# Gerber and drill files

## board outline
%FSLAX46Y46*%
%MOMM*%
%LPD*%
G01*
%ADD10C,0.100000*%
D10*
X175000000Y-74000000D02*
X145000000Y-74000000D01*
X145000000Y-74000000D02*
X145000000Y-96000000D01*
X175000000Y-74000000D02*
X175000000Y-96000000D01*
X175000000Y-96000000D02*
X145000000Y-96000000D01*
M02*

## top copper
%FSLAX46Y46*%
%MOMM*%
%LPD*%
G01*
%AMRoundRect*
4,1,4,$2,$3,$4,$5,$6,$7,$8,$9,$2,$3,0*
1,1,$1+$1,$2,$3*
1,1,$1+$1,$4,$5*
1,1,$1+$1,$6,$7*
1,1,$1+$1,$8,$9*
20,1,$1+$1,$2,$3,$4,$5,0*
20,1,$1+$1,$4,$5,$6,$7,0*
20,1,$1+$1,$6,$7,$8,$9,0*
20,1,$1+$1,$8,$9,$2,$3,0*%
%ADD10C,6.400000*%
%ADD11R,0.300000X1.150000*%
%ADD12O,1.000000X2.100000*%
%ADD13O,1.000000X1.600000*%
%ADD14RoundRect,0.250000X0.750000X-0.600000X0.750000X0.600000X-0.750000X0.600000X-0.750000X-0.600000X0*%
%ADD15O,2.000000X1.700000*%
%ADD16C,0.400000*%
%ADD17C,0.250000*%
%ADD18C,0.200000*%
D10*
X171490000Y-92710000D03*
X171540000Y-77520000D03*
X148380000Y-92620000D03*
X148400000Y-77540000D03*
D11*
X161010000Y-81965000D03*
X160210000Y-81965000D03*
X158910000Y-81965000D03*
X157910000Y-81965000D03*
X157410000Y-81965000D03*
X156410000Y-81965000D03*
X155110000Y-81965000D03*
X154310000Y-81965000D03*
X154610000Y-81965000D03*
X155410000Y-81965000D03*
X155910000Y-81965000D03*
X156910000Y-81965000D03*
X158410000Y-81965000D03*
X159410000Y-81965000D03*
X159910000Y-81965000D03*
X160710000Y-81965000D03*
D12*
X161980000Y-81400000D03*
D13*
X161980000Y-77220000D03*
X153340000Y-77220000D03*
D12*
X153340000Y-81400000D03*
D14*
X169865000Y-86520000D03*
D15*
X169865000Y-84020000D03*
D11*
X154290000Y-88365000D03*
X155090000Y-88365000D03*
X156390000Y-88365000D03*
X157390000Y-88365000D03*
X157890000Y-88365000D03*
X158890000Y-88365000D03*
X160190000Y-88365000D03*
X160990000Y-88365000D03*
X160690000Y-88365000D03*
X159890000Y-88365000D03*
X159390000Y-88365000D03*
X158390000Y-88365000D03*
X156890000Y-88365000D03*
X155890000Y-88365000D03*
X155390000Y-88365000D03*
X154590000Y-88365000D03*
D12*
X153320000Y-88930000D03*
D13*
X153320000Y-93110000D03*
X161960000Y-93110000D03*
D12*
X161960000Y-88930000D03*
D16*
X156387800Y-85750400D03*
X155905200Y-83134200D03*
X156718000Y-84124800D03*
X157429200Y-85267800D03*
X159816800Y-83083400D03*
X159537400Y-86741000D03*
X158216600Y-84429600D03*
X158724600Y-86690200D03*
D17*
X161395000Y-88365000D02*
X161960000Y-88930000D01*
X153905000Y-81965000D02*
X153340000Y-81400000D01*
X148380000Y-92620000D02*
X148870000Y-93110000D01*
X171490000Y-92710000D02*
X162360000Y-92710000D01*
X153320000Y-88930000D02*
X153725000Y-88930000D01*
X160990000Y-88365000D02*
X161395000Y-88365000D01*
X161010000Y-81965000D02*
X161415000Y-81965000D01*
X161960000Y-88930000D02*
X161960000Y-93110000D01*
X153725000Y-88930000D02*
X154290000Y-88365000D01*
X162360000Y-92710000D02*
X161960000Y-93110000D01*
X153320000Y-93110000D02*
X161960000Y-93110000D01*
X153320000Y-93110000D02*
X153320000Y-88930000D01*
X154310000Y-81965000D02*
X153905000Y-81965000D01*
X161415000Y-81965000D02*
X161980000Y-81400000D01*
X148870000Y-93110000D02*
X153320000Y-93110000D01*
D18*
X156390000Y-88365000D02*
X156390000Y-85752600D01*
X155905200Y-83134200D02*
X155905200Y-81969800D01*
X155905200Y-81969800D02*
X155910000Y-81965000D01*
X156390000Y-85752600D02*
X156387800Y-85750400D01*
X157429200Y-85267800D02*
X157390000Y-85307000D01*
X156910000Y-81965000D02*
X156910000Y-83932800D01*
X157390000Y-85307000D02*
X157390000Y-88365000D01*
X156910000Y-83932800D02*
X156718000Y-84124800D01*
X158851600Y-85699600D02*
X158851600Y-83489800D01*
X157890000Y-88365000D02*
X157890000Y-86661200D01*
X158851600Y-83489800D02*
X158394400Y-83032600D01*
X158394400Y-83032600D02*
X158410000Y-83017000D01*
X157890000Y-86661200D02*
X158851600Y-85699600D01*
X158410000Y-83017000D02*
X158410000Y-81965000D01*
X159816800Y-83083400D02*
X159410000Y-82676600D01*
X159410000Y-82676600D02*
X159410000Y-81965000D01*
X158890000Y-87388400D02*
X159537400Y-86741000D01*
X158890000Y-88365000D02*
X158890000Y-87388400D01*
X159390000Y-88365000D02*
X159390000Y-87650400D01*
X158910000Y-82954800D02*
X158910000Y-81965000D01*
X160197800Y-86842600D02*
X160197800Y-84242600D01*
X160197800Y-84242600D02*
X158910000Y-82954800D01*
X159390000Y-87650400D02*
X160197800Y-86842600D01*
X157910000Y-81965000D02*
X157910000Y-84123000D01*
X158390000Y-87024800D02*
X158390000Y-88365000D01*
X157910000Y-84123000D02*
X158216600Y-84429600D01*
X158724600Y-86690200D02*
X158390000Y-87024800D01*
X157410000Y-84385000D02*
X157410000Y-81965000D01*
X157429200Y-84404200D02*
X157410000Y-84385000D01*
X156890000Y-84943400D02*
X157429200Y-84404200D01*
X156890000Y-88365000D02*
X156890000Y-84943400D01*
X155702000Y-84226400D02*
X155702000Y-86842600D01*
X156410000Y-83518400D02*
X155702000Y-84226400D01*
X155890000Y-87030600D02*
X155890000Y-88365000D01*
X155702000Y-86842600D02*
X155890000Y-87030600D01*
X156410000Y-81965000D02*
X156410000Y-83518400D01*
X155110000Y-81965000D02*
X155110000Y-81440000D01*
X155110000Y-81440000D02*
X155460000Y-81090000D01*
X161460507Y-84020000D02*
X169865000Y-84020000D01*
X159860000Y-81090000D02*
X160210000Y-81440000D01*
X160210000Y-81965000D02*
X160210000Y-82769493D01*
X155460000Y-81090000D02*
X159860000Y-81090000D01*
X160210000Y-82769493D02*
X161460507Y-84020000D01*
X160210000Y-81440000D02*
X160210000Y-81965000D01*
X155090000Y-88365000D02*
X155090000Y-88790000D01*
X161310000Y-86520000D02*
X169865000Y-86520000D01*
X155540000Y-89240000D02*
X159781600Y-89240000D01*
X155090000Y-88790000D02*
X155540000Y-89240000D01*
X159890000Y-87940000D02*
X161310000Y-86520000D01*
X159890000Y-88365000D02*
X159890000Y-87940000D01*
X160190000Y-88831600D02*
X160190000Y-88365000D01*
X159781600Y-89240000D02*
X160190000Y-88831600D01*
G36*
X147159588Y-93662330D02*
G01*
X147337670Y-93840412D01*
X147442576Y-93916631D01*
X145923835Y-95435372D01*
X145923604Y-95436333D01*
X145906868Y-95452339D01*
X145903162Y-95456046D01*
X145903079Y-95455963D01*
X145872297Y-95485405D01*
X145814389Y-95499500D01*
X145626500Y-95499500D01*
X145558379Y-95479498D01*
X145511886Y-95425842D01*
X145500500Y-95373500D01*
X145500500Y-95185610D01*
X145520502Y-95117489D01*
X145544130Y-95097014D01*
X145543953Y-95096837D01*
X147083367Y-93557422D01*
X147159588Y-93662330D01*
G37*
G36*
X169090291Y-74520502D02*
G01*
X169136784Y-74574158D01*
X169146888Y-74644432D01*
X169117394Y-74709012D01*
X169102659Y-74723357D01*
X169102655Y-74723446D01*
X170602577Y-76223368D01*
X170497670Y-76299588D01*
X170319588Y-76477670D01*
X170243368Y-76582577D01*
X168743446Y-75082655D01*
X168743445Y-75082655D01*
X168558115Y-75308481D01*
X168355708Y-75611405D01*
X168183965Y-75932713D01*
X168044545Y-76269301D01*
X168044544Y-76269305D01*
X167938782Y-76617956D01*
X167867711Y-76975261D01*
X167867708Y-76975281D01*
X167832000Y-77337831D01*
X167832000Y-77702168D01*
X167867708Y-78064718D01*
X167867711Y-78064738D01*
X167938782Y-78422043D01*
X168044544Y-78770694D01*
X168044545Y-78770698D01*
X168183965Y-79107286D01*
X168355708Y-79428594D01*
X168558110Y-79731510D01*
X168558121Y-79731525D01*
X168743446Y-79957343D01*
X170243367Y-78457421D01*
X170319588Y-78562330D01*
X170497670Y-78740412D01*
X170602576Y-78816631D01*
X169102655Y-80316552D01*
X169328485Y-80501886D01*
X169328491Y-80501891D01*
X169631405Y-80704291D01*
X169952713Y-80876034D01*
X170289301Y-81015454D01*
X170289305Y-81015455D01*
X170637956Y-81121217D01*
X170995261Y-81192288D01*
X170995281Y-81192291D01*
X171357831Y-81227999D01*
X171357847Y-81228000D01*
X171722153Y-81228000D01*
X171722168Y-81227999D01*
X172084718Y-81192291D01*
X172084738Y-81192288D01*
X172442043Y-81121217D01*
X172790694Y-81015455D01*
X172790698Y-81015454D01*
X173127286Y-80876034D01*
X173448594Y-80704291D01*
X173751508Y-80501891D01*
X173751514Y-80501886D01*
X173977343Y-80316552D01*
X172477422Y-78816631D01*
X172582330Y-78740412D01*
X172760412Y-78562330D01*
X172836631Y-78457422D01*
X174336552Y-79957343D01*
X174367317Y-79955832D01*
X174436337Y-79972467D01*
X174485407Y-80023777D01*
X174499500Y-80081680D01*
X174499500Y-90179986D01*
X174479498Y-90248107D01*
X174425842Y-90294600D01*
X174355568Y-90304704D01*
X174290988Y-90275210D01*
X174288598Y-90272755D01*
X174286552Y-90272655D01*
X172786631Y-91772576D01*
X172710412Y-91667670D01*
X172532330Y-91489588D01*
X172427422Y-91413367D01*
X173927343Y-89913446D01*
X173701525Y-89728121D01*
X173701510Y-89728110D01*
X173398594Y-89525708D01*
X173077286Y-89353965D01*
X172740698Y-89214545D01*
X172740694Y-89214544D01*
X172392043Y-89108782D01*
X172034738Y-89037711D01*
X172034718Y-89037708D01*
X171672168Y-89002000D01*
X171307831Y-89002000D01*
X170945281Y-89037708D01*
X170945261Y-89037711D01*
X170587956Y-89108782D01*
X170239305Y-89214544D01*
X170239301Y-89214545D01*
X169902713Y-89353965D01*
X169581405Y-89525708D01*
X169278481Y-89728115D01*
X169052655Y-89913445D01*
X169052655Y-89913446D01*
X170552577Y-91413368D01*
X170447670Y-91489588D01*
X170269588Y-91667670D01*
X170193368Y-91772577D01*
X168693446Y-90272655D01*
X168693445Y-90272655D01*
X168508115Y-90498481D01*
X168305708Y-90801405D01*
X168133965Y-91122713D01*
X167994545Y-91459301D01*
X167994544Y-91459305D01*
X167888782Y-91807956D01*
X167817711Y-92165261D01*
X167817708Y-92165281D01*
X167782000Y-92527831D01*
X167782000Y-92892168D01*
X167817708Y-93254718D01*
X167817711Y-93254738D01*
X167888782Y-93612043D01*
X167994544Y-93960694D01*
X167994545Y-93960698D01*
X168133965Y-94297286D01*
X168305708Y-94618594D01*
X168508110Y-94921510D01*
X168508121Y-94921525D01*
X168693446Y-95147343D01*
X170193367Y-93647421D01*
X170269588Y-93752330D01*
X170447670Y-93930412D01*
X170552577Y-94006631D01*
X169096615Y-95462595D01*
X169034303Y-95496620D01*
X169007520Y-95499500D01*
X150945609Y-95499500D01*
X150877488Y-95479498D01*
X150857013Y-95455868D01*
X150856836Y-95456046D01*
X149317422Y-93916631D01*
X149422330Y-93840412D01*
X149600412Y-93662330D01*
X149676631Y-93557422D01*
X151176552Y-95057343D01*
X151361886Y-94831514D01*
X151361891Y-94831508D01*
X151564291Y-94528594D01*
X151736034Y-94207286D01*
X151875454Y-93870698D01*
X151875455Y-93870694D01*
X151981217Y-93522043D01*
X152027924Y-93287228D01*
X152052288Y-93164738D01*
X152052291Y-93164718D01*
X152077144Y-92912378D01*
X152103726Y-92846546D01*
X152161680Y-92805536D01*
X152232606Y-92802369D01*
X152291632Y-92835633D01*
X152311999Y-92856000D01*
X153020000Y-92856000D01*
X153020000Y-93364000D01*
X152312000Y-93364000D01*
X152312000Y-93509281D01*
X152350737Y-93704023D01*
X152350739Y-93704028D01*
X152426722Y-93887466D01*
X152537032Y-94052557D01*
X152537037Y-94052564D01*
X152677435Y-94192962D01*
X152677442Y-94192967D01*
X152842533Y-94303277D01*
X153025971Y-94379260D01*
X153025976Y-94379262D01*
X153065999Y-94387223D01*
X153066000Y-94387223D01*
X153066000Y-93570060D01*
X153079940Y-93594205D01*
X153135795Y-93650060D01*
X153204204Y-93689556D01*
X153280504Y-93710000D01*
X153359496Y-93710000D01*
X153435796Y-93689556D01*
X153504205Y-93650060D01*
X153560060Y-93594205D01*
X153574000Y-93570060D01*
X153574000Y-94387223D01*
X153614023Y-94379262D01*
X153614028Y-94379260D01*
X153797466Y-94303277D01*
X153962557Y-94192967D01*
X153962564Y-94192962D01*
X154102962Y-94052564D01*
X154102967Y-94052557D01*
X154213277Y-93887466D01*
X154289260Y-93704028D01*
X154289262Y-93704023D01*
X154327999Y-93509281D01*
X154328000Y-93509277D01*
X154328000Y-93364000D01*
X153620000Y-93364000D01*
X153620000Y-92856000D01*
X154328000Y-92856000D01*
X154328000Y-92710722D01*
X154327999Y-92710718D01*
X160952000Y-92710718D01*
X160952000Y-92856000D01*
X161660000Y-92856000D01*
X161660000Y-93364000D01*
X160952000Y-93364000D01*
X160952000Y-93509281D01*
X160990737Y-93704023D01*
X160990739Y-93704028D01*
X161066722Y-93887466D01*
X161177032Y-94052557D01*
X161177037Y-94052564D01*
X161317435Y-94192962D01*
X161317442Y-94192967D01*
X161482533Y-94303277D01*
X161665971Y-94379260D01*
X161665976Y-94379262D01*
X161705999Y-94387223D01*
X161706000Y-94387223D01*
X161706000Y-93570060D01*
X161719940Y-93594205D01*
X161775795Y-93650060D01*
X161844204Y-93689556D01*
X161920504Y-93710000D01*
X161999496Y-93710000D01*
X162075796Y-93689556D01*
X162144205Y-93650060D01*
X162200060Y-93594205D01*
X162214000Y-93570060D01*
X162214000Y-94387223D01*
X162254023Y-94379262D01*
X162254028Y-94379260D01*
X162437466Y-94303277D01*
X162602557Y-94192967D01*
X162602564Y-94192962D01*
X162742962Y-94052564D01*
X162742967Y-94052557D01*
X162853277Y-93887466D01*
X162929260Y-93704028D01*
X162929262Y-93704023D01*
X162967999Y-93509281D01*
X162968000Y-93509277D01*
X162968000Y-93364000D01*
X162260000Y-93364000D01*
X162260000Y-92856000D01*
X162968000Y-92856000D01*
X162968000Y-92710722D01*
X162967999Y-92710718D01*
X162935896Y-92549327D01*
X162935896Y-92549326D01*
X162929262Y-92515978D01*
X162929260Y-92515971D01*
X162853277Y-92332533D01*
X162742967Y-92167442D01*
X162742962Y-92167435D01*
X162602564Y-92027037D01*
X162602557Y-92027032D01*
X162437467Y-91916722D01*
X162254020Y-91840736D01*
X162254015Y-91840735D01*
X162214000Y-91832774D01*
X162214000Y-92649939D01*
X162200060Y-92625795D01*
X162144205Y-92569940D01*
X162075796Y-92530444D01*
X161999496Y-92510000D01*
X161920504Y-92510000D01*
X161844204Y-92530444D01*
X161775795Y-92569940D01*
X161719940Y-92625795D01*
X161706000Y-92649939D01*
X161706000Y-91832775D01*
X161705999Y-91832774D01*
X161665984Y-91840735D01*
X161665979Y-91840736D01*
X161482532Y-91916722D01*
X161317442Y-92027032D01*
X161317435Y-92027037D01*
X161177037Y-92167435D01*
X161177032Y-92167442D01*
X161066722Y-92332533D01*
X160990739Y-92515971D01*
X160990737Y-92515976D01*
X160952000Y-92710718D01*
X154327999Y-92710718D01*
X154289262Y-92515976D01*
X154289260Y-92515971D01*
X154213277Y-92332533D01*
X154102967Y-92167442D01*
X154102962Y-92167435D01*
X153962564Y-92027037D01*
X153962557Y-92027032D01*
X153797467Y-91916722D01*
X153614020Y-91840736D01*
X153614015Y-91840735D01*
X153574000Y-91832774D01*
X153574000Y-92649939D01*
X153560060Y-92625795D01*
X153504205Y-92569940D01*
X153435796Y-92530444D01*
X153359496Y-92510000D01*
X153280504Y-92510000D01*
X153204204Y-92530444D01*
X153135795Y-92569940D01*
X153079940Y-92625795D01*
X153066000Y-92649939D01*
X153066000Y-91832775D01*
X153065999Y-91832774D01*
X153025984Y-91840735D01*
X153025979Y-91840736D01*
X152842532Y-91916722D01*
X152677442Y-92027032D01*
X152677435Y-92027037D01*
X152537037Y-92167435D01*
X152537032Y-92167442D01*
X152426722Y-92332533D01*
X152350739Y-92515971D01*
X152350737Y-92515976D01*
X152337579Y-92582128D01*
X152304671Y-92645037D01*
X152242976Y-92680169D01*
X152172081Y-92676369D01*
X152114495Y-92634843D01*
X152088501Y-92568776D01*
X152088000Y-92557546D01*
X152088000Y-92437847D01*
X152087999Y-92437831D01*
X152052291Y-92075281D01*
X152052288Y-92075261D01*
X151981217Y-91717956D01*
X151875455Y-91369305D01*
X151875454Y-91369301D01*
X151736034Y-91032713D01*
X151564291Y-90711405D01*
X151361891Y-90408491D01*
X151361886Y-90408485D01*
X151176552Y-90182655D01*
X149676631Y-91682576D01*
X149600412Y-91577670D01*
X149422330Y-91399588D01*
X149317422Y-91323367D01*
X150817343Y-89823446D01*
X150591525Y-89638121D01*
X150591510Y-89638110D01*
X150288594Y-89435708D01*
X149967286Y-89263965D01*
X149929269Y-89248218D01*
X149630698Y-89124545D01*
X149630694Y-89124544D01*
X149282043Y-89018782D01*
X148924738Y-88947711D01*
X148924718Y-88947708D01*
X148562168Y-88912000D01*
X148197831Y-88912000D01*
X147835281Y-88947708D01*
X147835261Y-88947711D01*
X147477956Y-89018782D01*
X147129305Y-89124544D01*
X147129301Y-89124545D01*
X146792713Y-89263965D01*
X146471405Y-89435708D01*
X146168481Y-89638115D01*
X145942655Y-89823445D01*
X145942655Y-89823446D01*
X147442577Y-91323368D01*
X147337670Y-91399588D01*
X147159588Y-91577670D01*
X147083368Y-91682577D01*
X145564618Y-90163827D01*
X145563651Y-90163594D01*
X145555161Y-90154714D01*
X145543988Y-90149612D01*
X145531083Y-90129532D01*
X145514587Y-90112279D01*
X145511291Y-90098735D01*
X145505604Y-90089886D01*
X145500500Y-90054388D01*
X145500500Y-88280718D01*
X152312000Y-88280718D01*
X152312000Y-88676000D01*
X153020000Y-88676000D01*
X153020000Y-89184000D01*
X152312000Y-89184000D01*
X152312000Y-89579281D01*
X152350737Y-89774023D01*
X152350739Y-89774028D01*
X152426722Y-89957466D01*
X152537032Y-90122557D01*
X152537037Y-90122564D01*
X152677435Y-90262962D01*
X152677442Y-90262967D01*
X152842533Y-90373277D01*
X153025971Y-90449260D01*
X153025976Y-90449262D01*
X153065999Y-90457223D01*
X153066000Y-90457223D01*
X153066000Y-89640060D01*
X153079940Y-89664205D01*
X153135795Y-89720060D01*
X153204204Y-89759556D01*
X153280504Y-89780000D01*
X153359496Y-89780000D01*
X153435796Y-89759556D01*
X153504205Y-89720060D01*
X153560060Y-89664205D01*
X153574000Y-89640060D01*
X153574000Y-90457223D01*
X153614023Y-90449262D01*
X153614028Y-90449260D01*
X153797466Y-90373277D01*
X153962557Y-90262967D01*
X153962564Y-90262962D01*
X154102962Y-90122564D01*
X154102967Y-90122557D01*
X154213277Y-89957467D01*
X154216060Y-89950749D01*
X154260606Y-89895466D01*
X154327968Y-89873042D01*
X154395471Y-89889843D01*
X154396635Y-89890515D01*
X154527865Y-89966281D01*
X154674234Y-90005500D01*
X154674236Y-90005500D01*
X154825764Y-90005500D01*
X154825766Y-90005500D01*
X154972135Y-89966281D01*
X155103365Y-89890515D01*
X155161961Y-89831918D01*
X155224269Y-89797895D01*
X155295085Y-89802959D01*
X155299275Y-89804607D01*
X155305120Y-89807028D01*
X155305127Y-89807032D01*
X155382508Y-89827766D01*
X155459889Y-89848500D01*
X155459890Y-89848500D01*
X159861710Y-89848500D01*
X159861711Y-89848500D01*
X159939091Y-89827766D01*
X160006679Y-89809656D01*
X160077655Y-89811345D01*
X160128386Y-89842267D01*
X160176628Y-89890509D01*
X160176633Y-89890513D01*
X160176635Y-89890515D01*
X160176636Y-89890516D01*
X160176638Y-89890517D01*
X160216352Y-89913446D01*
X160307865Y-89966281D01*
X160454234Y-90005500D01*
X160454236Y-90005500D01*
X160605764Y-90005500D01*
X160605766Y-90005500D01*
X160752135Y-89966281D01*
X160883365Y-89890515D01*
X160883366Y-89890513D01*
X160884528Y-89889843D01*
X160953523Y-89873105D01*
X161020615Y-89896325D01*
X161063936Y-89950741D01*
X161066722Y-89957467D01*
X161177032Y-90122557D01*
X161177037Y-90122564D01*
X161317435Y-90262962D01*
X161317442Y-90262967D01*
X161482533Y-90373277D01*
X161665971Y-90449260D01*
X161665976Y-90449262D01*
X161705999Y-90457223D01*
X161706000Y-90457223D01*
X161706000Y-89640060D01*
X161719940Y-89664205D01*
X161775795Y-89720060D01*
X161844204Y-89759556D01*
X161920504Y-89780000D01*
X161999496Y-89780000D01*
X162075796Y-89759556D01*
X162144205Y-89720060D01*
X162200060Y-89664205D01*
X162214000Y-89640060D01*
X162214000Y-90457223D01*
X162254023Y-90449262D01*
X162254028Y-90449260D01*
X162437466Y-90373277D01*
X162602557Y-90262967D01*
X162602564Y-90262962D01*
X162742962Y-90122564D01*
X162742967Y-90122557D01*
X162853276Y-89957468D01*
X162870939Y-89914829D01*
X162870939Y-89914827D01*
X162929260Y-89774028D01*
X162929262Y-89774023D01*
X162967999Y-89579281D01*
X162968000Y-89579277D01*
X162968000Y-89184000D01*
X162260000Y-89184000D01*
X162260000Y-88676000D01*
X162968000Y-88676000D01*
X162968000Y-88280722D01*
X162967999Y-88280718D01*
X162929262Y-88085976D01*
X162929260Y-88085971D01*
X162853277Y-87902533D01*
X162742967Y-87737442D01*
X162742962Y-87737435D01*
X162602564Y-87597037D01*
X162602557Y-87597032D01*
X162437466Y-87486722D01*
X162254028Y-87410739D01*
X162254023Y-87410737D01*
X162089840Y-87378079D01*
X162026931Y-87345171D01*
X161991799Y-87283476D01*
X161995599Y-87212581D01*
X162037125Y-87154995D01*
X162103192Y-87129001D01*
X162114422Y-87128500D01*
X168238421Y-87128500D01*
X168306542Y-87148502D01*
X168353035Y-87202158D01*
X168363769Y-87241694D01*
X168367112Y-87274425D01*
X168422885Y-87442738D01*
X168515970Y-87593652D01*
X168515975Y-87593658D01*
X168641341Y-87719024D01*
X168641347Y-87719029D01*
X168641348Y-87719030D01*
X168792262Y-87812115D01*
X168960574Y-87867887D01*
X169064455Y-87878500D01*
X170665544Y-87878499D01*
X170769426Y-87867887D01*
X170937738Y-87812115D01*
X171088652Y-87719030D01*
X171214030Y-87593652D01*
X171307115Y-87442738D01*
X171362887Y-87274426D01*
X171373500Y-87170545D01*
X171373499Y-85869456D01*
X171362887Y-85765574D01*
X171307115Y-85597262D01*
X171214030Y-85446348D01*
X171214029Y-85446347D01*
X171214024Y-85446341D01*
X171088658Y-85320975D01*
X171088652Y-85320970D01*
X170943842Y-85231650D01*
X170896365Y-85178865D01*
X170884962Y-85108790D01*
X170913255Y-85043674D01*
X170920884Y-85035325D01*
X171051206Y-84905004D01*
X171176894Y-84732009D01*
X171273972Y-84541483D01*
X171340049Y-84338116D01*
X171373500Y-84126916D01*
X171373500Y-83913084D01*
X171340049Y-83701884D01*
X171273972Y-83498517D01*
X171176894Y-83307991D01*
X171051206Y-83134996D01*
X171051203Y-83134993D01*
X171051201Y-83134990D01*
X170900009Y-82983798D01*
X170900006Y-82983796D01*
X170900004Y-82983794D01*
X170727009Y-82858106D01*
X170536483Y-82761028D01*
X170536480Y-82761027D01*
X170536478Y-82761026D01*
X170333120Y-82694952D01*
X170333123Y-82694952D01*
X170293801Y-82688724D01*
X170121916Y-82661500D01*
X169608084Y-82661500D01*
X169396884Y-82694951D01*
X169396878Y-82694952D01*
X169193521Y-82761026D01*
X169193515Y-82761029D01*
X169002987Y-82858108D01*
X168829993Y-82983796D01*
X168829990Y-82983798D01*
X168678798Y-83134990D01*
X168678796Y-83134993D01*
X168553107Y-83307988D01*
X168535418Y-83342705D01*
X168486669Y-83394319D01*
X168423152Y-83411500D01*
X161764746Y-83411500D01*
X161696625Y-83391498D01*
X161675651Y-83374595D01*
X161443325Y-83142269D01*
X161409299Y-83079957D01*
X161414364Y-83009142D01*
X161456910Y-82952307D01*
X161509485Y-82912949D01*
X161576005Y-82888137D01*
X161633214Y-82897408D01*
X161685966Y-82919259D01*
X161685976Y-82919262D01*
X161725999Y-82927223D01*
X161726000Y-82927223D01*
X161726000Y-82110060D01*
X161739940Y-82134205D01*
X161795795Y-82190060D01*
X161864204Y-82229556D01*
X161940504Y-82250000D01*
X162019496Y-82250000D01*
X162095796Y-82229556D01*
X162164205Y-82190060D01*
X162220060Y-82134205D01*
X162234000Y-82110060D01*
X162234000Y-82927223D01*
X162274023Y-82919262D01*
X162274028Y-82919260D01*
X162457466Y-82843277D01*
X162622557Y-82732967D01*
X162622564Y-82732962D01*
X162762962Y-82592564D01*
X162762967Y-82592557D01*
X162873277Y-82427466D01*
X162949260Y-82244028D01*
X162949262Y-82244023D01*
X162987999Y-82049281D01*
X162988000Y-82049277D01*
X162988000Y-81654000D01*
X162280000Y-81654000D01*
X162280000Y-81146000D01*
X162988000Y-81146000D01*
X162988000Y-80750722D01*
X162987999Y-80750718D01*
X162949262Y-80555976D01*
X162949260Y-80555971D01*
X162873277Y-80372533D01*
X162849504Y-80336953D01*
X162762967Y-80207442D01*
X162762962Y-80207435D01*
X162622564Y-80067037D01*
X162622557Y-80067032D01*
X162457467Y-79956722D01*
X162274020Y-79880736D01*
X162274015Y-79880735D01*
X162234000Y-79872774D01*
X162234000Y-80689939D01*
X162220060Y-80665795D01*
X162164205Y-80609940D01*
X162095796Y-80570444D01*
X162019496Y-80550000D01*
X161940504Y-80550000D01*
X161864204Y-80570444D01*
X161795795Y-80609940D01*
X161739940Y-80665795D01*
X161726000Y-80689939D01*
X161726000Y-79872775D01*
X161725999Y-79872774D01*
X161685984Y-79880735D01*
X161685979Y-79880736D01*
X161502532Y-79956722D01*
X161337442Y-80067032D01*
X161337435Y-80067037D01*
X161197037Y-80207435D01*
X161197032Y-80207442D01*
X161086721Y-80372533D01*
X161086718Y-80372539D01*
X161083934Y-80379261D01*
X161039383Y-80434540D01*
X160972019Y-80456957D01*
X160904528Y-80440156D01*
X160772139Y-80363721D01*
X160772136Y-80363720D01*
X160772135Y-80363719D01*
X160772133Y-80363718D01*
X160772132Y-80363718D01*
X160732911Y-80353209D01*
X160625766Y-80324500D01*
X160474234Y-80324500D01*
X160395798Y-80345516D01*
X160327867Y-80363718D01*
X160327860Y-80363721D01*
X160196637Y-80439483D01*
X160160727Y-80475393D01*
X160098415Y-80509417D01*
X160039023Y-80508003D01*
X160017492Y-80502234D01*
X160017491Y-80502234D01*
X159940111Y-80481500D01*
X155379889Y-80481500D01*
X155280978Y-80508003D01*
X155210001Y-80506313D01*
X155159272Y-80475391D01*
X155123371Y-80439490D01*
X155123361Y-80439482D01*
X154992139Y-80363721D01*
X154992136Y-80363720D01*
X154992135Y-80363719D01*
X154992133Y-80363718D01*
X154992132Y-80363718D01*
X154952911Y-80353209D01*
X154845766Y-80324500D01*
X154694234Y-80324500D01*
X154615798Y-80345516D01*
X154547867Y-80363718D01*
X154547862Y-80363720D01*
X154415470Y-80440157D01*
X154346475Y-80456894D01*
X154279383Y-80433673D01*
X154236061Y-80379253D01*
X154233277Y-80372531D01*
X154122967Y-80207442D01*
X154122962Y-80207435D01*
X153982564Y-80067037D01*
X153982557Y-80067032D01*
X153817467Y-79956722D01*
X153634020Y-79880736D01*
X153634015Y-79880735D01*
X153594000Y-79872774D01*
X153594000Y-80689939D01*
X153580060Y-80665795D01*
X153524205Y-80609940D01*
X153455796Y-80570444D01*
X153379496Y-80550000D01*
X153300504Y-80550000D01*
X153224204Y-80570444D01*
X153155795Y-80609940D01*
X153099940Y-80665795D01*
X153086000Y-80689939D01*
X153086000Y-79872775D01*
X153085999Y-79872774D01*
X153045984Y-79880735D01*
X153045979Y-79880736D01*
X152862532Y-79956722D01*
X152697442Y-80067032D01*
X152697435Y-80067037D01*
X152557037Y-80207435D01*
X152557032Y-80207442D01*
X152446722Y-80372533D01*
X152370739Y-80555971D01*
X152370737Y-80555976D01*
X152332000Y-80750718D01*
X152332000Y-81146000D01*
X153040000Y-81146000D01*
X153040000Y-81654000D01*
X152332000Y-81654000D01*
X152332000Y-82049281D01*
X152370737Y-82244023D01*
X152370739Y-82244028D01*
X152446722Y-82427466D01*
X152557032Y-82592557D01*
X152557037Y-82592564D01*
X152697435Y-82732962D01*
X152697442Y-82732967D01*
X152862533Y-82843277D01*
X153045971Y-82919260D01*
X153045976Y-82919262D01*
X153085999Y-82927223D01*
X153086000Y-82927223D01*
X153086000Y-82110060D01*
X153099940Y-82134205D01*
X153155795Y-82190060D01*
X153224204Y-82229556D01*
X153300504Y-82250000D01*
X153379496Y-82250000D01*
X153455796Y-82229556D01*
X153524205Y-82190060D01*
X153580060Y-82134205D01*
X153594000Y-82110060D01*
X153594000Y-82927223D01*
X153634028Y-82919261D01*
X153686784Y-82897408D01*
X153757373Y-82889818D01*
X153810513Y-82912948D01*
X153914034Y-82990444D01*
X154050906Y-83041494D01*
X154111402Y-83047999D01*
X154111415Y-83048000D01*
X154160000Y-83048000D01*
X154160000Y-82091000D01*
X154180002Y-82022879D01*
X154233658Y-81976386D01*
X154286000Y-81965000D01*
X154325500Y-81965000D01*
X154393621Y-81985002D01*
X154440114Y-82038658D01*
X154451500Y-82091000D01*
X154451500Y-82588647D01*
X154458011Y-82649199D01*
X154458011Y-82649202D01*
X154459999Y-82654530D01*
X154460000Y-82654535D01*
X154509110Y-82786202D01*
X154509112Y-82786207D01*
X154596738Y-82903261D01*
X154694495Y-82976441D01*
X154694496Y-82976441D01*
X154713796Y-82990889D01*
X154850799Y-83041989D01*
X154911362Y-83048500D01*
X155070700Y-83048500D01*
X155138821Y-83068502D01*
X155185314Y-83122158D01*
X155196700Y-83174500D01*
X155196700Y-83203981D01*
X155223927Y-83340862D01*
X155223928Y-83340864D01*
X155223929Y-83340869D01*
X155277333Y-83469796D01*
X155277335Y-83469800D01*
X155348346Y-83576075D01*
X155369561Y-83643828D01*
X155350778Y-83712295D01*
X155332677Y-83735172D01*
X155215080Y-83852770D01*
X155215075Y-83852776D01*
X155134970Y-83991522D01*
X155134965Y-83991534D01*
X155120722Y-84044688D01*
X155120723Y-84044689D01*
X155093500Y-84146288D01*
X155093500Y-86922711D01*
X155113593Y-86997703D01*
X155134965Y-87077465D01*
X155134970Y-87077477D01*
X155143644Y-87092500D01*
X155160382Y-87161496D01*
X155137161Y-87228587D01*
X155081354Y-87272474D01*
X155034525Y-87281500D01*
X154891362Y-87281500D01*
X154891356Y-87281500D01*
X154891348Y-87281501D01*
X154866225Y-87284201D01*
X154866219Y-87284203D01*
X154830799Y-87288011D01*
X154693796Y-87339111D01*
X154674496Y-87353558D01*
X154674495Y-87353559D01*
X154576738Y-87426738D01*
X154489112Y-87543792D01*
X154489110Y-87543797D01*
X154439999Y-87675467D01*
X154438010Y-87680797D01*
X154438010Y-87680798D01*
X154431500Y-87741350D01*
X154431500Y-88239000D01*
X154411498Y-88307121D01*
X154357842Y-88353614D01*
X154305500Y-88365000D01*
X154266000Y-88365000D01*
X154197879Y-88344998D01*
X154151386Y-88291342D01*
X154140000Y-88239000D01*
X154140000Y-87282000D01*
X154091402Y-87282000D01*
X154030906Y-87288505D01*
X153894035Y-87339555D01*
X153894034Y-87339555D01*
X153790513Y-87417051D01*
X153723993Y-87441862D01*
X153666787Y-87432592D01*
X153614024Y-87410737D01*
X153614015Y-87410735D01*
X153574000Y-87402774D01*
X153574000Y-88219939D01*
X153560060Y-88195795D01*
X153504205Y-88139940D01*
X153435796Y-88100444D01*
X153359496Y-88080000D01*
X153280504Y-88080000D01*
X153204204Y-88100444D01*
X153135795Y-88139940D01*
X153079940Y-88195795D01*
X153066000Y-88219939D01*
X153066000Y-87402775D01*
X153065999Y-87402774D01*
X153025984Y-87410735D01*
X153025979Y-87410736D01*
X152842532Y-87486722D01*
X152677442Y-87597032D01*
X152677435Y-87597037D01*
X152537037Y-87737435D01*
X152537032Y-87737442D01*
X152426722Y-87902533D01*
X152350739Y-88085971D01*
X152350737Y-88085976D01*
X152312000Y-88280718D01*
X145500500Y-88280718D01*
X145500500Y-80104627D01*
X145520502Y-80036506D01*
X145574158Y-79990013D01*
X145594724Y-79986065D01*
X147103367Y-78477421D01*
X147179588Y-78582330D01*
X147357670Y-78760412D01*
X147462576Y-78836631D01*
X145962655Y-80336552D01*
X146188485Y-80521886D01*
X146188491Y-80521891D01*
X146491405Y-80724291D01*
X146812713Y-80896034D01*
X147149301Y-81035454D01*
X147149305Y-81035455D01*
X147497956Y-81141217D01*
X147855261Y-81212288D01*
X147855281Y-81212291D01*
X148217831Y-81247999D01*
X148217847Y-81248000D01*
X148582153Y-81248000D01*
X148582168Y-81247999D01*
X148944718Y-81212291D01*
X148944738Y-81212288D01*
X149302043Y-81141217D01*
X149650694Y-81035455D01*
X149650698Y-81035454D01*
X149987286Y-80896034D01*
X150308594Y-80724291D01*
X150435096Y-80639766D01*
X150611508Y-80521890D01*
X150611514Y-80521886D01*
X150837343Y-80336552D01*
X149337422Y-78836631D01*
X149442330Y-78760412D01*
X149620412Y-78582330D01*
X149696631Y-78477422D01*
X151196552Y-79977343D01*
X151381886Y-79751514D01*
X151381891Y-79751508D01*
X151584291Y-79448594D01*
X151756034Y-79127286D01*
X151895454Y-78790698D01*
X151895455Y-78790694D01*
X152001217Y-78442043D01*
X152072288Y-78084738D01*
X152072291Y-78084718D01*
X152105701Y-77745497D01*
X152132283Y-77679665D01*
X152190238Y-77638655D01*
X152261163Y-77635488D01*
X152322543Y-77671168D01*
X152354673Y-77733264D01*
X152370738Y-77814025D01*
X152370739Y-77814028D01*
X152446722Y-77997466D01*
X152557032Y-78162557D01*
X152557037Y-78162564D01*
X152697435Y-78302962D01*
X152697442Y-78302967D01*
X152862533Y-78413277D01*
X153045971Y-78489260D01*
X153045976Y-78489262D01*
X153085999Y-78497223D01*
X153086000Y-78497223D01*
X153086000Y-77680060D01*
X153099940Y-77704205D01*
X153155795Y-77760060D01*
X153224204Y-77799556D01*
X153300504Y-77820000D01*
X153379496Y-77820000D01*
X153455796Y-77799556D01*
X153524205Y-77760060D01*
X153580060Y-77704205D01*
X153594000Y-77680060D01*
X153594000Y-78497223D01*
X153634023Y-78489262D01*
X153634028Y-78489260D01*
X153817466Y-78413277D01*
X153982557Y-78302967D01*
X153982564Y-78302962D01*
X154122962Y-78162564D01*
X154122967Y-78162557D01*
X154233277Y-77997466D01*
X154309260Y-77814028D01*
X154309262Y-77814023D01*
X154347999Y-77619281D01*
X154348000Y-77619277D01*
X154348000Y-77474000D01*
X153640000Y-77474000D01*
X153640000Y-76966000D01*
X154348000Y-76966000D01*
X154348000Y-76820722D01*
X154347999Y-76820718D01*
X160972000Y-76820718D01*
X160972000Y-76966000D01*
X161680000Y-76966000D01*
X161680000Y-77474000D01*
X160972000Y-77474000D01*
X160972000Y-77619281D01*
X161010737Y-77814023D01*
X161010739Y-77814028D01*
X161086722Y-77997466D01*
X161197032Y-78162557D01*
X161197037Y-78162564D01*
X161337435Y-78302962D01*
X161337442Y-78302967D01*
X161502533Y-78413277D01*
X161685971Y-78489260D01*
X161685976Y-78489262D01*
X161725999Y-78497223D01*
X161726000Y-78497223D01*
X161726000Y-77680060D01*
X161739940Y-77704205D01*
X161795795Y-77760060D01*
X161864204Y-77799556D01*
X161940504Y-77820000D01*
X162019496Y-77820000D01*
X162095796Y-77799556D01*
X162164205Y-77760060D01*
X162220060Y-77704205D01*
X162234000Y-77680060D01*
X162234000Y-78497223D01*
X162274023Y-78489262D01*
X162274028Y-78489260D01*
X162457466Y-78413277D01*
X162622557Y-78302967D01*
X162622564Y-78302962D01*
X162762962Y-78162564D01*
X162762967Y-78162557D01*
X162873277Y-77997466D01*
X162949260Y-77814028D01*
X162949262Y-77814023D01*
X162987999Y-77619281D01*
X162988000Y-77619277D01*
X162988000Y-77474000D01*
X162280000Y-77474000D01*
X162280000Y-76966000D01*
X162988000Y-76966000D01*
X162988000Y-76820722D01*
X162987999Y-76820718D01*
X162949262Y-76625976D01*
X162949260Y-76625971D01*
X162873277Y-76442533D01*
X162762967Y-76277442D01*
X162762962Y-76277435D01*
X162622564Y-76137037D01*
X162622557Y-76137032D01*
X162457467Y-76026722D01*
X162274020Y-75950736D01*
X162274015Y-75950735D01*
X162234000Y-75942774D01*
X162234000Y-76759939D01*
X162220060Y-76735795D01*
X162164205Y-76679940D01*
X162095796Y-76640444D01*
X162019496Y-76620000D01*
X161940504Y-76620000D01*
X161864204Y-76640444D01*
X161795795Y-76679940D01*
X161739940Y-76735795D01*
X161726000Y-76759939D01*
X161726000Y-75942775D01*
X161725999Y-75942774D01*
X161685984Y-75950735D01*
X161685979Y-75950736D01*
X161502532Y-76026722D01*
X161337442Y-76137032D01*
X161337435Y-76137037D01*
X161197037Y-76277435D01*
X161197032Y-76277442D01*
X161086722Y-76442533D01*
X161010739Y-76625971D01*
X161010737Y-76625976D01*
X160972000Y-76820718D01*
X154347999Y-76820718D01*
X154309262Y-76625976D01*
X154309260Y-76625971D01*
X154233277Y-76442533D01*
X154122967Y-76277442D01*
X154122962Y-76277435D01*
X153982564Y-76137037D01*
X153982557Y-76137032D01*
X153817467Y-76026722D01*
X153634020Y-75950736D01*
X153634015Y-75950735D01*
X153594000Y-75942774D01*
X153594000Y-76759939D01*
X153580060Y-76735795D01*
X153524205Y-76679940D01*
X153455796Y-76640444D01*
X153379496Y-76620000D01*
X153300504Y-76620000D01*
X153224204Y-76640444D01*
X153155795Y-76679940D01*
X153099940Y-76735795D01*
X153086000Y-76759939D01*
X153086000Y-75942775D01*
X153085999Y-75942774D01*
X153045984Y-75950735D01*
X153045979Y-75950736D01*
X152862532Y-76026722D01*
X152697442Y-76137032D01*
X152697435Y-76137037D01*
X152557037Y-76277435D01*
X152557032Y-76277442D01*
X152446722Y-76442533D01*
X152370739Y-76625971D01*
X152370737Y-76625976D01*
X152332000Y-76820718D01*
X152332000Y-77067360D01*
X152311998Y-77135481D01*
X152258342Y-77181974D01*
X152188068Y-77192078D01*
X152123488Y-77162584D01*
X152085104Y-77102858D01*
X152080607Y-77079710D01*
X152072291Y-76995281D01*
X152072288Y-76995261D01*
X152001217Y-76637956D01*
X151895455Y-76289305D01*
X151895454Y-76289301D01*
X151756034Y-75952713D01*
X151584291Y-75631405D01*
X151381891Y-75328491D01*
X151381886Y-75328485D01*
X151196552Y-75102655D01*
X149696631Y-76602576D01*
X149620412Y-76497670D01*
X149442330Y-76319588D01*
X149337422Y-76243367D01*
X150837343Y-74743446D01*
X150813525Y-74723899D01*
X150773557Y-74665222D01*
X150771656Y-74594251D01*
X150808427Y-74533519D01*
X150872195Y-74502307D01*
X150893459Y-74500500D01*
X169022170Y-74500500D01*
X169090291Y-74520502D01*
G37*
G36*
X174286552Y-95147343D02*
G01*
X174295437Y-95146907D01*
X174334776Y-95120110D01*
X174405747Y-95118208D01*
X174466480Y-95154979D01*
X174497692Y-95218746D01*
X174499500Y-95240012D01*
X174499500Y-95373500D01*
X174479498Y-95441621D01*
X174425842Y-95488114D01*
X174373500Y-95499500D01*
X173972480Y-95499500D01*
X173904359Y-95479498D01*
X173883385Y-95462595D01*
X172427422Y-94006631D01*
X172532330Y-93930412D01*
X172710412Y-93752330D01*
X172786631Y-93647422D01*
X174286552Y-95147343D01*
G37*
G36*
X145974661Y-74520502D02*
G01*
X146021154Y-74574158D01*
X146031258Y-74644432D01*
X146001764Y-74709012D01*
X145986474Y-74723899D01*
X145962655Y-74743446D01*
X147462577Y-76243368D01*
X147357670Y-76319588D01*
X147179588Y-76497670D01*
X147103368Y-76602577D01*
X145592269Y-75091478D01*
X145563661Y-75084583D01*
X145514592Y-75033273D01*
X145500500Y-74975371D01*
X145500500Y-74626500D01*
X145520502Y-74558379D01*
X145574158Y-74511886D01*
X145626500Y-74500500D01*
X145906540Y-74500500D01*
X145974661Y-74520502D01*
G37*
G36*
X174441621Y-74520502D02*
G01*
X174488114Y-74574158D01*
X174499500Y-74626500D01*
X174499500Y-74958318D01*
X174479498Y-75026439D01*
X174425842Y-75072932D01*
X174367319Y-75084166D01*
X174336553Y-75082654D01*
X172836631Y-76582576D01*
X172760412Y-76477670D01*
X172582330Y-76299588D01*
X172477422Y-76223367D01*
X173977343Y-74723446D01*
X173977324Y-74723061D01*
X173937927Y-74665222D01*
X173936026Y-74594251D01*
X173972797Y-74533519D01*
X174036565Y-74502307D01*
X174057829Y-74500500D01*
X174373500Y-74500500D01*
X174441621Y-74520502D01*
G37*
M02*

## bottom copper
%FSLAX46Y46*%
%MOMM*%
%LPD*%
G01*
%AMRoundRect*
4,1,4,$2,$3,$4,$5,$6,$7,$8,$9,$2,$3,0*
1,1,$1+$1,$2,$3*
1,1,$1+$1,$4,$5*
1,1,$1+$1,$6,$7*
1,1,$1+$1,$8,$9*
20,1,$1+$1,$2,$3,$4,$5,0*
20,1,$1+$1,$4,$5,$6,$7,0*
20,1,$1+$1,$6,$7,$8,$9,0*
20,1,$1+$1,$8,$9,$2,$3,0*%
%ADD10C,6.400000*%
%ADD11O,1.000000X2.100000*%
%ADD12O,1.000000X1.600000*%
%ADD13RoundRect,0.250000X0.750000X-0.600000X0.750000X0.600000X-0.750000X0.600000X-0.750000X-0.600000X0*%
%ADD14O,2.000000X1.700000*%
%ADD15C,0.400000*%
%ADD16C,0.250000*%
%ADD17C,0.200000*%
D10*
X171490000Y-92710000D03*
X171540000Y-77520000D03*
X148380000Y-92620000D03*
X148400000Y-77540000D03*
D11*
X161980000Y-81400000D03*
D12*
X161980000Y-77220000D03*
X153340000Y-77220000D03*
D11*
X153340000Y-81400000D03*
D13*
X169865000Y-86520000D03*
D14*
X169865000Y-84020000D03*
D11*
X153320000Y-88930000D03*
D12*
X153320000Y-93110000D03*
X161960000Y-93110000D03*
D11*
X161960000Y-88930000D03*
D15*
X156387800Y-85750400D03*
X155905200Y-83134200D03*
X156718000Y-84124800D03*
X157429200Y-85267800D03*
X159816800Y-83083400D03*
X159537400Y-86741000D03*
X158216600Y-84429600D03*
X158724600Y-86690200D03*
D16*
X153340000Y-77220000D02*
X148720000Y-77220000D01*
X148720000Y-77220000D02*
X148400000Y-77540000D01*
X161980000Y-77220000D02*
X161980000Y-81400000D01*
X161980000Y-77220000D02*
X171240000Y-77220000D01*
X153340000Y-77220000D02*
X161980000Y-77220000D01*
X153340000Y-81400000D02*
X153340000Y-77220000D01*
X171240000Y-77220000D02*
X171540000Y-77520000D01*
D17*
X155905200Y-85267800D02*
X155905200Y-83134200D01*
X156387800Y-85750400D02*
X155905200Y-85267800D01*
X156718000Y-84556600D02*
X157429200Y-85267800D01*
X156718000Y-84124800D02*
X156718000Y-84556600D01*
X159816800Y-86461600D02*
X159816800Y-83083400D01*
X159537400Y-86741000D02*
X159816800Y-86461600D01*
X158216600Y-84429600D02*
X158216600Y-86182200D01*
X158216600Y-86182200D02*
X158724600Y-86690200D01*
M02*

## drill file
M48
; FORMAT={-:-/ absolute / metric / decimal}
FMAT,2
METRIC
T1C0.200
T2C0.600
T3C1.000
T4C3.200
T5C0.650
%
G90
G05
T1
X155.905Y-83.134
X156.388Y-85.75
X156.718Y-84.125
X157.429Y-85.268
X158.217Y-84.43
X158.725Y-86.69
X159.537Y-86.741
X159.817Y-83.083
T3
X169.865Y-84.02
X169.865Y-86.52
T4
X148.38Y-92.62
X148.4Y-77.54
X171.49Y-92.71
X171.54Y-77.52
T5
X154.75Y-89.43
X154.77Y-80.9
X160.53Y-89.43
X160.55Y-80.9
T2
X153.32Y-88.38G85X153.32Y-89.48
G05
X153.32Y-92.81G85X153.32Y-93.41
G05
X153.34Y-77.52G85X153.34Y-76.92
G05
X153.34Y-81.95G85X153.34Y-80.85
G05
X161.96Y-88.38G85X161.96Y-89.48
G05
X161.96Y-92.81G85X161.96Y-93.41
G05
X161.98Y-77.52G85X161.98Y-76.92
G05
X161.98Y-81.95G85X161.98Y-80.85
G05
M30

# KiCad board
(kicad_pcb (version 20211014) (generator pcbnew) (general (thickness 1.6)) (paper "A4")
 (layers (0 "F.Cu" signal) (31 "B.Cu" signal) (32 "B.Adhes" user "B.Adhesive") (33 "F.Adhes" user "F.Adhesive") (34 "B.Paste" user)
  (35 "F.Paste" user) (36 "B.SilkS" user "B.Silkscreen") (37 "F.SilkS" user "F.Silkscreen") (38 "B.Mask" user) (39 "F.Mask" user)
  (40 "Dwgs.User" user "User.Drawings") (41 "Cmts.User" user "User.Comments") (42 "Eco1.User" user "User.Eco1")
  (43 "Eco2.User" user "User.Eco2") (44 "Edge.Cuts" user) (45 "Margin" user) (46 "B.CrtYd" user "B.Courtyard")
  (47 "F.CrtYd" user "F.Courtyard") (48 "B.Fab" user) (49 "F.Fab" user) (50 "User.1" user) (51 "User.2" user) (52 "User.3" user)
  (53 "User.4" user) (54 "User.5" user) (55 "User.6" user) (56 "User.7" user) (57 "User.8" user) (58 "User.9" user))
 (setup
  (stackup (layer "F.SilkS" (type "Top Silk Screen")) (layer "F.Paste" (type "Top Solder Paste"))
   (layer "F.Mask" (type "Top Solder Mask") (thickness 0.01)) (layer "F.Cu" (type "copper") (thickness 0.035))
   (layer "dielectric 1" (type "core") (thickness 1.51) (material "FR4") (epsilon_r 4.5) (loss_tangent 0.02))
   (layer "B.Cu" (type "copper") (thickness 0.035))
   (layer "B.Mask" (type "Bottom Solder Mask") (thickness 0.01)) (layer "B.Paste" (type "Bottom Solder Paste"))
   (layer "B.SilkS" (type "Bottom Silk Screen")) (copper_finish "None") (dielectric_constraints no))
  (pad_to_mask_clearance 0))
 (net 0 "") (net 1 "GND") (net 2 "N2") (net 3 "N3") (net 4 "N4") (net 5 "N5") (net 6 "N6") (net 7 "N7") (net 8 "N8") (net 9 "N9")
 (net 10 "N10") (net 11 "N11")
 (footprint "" (layer "F.Cu") (at 171.49 92.71)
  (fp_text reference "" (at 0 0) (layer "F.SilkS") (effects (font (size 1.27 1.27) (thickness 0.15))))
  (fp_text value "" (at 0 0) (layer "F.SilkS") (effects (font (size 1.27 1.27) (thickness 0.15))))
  (pad "1" thru_hole circle locked (at 0 0) (size 6.4 6.4) (drill 3.2) (layers *.Cu *.Mask) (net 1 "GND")))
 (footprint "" (layer "F.Cu") (at 171.54 77.52)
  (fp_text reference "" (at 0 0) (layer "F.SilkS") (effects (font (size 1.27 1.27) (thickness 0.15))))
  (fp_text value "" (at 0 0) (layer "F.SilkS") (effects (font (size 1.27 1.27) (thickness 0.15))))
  (pad "1" thru_hole circle locked (at 0 0) (size 6.4 6.4) (drill 3.2) (layers *.Cu *.Mask) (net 1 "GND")))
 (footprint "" (layer "F.Cu") (at 148.38 92.62)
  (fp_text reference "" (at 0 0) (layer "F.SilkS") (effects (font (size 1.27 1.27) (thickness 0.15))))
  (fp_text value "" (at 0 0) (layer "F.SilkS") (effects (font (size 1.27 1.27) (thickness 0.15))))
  (pad "1" thru_hole circle locked (at 0 0) (size 6.4 6.4) (drill 3.2) (layers *.Cu *.Mask) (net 1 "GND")))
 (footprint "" (layer "F.Cu") (at 148.4 77.54)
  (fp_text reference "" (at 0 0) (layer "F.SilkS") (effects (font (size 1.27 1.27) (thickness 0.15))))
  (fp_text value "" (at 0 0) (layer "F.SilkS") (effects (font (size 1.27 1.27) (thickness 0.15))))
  (pad "1" thru_hole circle locked (at 0 0) (size 6.4 6.4) (drill 3.2) (layers *.Cu *.Mask) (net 1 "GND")))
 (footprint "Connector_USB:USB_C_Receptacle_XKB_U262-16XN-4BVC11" (layer "F.Cu") (at 157.66 78.295 180)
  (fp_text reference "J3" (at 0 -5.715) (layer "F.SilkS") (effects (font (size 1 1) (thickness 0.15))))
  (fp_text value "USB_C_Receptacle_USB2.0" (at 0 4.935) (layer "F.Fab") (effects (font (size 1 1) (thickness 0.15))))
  (pad "" np_thru_hole circle (at 2.89 -2.605 180) (size 0.65 0.65) (drill 0.65) (layers *.Cu *.Mask))
  (pad "" np_thru_hole circle (at -2.89 -2.605 180) (size 0.65 0.65) (drill 0.65) (layers *.Cu *.Mask))
  (pad "A1" smd rect (at -3.35 -3.67 180) (size 0.3 1.15) (layers "F.Cu" "F.Paste" "F.Mask") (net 1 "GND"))
  (pad "A4" smd rect (at -2.55 -3.67 180) (size 0.3 1.15) (layers "F.Cu" "F.Paste" "F.Mask") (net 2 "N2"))
  (pad "A5" smd rect (at -1.25 -3.67 180) (size 0.3 1.15) (layers "F.Cu" "F.Paste" "F.Mask") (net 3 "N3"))
  (pad "A6" smd rect (at -0.25 -3.67 180) (size 0.3 1.15) (layers "F.Cu" "F.Paste" "F.Mask") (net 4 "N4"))
  (pad "A7" smd rect (at 0.25 -3.67 180) (size 0.3 1.15) (layers "F.Cu" "F.Paste" "F.Mask") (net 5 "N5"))
  (pad "A8" smd rect locked (at 1.25 -3.67 180) (size 0.3 1.15) (layers "F.Cu" "F.Paste" "F.Mask") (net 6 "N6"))
  (pad "A9" smd rect (at 2.55 -3.67 180) (size 0.3 1.15) (layers "F.Cu" "F.Paste" "F.Mask") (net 2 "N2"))
  (pad "A12" smd rect (at 3.35 -3.67 180) (size 0.3 1.15) (layers "F.Cu" "F.Paste" "F.Mask") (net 1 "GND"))
  (pad "B1" smd rect (at 3.05 -3.67 180) (size 0.3 1.15) (layers "F.Cu" "F.Paste" "F.Mask") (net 1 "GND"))
  (pad "B4" smd rect (at 2.25 -3.67 180) (size 0.3 1.15) (layers "F.Cu" "F.Paste" "F.Mask") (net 2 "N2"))
  (pad "B5" smd rect (at 1.75 -3.67 180) (size 0.3 1.15) (layers "F.Cu" "F.Paste" "F.Mask") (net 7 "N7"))
  (pad "B6" smd rect (at 0.75 -3.67 180) (size 0.3 1.15) (layers "F.Cu" "F.Paste" "F.Mask") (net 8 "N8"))
  (pad "B7" smd rect (at -0.75 -3.67 180) (size 0.3 1.15) (layers "F.Cu" "F.Paste" "F.Mask") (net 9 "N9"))
  (pad "B8" smd rect (at -1.75 -3.67 180) (size 0.3 1.15) (layers "F.Cu" "F.Paste" "F.Mask") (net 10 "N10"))
  (pad "B9" smd rect (at -2.25 -3.67 180) (size 0.3 1.15) (layers "F.Cu" "F.Paste" "F.Mask") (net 2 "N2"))
  (pad "B12" smd rect (at -3.05 -3.67 180) (size 0.3 1.15) (layers "F.Cu" "F.Paste" "F.Mask") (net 1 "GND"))
  (pad "S1" thru_hole oval (at -4.32 -3.105 180) (size 1 2.1) (drill oval 0.6 1.7) (layers *.Cu *.Mask) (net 1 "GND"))
  (pad "S1" thru_hole oval (at -4.32 1.075 180) (size 1 1.6) (drill oval 0.6 1.2) (layers *.Cu *.Mask) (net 1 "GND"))
  (pad "S1" thru_hole oval (at 4.32 1.075 180) (size 1 1.6) (drill oval 0.6 1.2) (layers *.Cu *.Mask) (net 1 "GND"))
  (pad "S1" thru_hole oval (at 4.32 -3.105 180) (size 1 2.1) (drill oval 0.6 1.7) (layers *.Cu *.Mask) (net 1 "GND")))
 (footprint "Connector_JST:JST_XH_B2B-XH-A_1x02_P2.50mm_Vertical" (layer "F.Cu") (at 169.865 86.52 90)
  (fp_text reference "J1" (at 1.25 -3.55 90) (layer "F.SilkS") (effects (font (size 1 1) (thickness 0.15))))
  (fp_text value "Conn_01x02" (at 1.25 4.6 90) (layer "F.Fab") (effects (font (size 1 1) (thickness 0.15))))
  (pad "1" thru_hole roundrect (at 0 0 90) (size 1.7 2) (drill 1) (layers *.Cu *.Mask) (roundrect_rratio 0.147059) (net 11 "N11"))
  (pad "2" thru_hole oval (at 2.5 0 90) (size 1.7 2) (drill 1) (layers *.Cu *.Mask) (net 2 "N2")))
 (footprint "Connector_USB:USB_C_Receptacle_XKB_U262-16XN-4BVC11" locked (layer "F.Cu") (at 157.64 92.035)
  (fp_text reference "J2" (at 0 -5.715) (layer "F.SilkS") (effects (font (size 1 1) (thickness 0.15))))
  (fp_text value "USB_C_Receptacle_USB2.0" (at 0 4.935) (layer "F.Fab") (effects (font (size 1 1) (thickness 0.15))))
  (pad "" np_thru_hole circle locked (at 2.89 -2.605) (size 0.65 0.65) (drill 0.65) (layers *.Cu *.Mask))
  (pad "" np_thru_hole circle locked (at -2.89 -2.605) (size 0.65 0.65) (drill 0.65) (layers *.Cu *.Mask))
  (pad "A1" smd rect locked (at -3.35 -3.67) (size 0.3 1.15) (layers "F.Cu" "F.Paste" "F.Mask") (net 1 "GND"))
  (pad "A4" smd rect locked (at -2.55 -3.67) (size 0.3 1.15) (layers "F.Cu" "F.Paste" "F.Mask") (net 11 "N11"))
  (pad "A5" smd rect locked (at -1.25 -3.67) (size 0.3 1.15) (layers "F.Cu" "F.Paste" "F.Mask") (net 7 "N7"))
  (pad "A6" smd rect locked (at -0.25 -3.67) (size 0.3 1.15) (layers "F.Cu" "F.Paste" "F.Mask") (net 8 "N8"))
  (pad "A7" smd rect locked (at 0.25 -3.67) (size 0.3 1.15) (layers "F.Cu" "F.Paste" "F.Mask") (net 9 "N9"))
  (pad "A8" smd rect locked (at 1.25 -3.67) (size 0.3 1.15) (layers "F.Cu" "F.Paste" "F.Mask") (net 10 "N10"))
  (pad "A9" smd rect locked (at 2.55 -3.67) (size 0.3 1.15) (layers "F.Cu" "F.Paste" "F.Mask") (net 11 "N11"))
  (pad "A12" smd rect locked (at 3.35 -3.67) (size 0.3 1.15) (layers "F.Cu" "F.Paste" "F.Mask") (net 1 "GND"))
  (pad "B1" smd rect locked (at 3.05 -3.67) (size 0.3 1.15) (layers "F.Cu" "F.Paste" "F.Mask") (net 1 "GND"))
  (pad "B4" smd rect locked (at 2.25 -3.67) (size 0.3 1.15) (layers "F.Cu" "F.Paste" "F.Mask") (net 11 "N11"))
  (pad "B5" smd rect locked (at 1.75 -3.67) (size 0.3 1.15) (layers "F.Cu" "F.Paste" "F.Mask") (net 3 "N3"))
  (pad "B6" smd rect locked (at 0.75 -3.67) (size 0.3 1.15) (layers "F.Cu" "F.Paste" "F.Mask") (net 4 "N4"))
  (pad "B7" smd rect locked (at -0.75 -3.67) (size 0.3 1.15) (layers "F.Cu" "F.Paste" "F.Mask") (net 5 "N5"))
  (pad "B8" smd rect locked (at -1.75 -3.67) (size 0.3 1.15) (layers "F.Cu" "F.Paste" "F.Mask") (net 6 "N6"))
  (pad "B9" smd rect locked (at -2.25 -3.67) (size 0.3 1.15) (layers "F.Cu" "F.Paste" "F.Mask") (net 11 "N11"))
  (pad "B12" smd rect locked (at -3.05 -3.67) (size 0.3 1.15) (layers "F.Cu" "F.Paste" "F.Mask") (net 1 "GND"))
  (pad "S1" thru_hole oval locked (at -4.32 -3.105) (size 1 2.1) (drill oval 0.6 1.7) (layers *.Cu *.Mask) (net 1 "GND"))
  (pad "S1" thru_hole oval locked (at -4.32 1.075) (size 1 1.6) (drill oval 0.6 1.2) (layers *.Cu *.Mask) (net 1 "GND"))
  (pad "S1" thru_hole oval locked (at 4.32 1.075) (size 1 1.6) (drill oval 0.6 1.2) (layers *.Cu *.Mask) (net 1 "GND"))
  (pad "S1" thru_hole oval locked (at 4.32 -3.105) (size 1 2.1) (drill oval 0.6 1.7) (layers *.Cu *.Mask) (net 1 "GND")))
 (gr_line (start 175 74) (end 145 74) (layer "Edge.Cuts") (width 0.1))
 (gr_line (start 145 74) (end 145 96) (layer "Edge.Cuts") (width 0.1))
 (gr_line (start 175 74) (end 175 96) (layer "Edge.Cuts") (width 0.1))
 (gr_line (start 175 96) (end 145 96) (layer "Edge.Cuts") (width 0.1))
 (segment (start 161.395 88.365) (end 161.96 88.93) (width 0.25) (layer "F.Cu") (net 1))
 (segment (start 153.905 81.965) (end 153.34 81.4) (width 0.25) (layer "F.Cu") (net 1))
 (segment (start 148.38 92.62) (end 148.87 93.11) (width 0.25) (layer "F.Cu") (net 1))
 (segment (start 171.49 92.71) (end 162.36 92.71) (width 0.25) (layer "F.Cu") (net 1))
 (segment (start 153.32 88.93) (end 153.725 88.93) (width 0.25) (layer "F.Cu") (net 1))
 (segment (start 160.99 88.365) (end 161.395 88.365) (width 0.25) (layer "F.Cu") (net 1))
 (segment (start 161.01 81.965) (end 161.415 81.965) (width 0.25) (layer "F.Cu") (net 1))
 (segment (start 161.96 88.93) (end 161.96 93.11) (width 0.25) (layer "F.Cu") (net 1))
 (segment (start 153.725 88.93) (end 154.29 88.365) (width 0.25) (layer "F.Cu") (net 1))
 (segment (start 162.36 92.71) (end 161.96 93.11) (width 0.25) (layer "F.Cu") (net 1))
 (segment (start 153.32 93.11) (end 161.96 93.11) (width 0.25) (layer "F.Cu") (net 1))
 (segment (start 153.32 93.11) (end 153.32 88.93) (width 0.25) (layer "F.Cu") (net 1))
 (segment (start 154.31 81.965) (end 153.905 81.965) (width 0.25) (layer "F.Cu") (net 1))
 (segment (start 161.415 81.965) (end 161.98 81.4) (width 0.25) (layer "F.Cu") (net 1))
 (segment (start 148.87 93.11) (end 153.32 93.11) (width 0.25) (layer "F.Cu") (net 1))
 (segment (start 153.34 77.22) (end 148.72 77.22) (width 0.25) (layer "B.Cu") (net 1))
 (segment (start 148.72 77.22) (end 148.4 77.54) (width 0.25) (layer "B.Cu") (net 1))
 (segment (start 161.98 77.22) (end 161.98 81.4) (width 0.25) (layer "B.Cu") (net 1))
 (segment (start 161.98 77.22) (end 171.24 77.22) (width 0.25) (layer "B.Cu") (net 1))
 (segment (start 153.34 77.22) (end 161.98 77.22) (width 0.25) (layer "B.Cu") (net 1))
 (segment (start 153.34 81.4) (end 153.34 77.22) (width 0.25) (layer "B.Cu") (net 1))
 (segment (start 171.24 77.22) (end 171.54 77.52) (width 0.25) (layer "B.Cu") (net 1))
 (segment (start 156.39 88.365) (end 156.39 85.7526) (width 0.2) (layer "F.Cu") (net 7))
 (segment (start 155.9052 83.1342) (end 155.9052 81.9698) (width 0.2) (layer "F.Cu") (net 7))
 (segment (start 155.9052 81.9698) (end 155.91 81.965) (width 0.2) (layer "F.Cu") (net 7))
 (segment (start 156.39 85.7526) (end 156.3878 85.7504) (width 0.2) (layer "F.Cu") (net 7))
 (via (at 156.3878 85.7504) (size 0.4) (drill 0.2) (layers "F.Cu" "B.Cu") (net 7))
 (via (at 155.9052 83.1342) (size 0.4) (drill 0.2) (layers "F.Cu" "B.Cu") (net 7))
 (segment (start 155.9052 85.2678) (end 155.9052 83.1342) (width 0.2) (layer "B.Cu") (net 7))
 (segment (start 156.3878 85.7504) (end 155.9052 85.2678) (width 0.2) (layer "B.Cu") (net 7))
 (segment (start 157.4292 85.2678) (end 157.39 85.307) (width 0.2) (layer "F.Cu") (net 8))
 (segment (start 156.91 81.965) (end 156.91 83.9328) (width 0.2) (layer "F.Cu") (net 8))
 (segment (start 157.39 85.307) (end 157.39 88.365) (width 0.2) (layer "F.Cu") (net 8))
 (segment (start 156.91 83.9328) (end 156.718 84.1248) (width 0.2) (layer "F.Cu") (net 8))
 (via (at 156.718 84.1248) (size 0.4) (drill 0.2) (layers "F.Cu" "B.Cu") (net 8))
 (via (at 157.4292 85.2678) (size 0.4) (drill 0.2) (layers "F.Cu" "B.Cu") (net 8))
 (segment (start 156.718 84.5566) (end 157.4292 85.2678) (width 0.2) (layer "B.Cu") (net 8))
 (segment (start 156.718 84.1248) (end 156.718 84.5566) (width 0.2) (layer "B.Cu") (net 8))
 (segment (start 158.8516 85.6996) (end 158.8516 83.4898) (width 0.2) (layer "F.Cu") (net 9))
 (segment (start 157.89 88.365) (end 157.89 86.6612) (width 0.2) (layer "F.Cu") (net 9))
 (segment (start 158.8516 83.4898) (end 158.3944 83.0326) (width 0.2) (layer "F.Cu") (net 9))
 (segment (start 158.3944 83.0326) (end 158.41 83.017) (width 0.2) (layer "F.Cu") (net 9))
 (segment (start 157.89 86.6612) (end 158.8516 85.6996) (width 0.2) (layer "F.Cu") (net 9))
 (segment (start 158.41 83.017) (end 158.41 81.965) (width 0.2) (layer "F.Cu") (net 9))
 (segment (start 159.8168 83.0834) (end 159.41 82.6766) (width 0.2) (layer "F.Cu") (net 10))
 (segment (start 159.41 82.6766) (end 159.41 81.965) (width 0.2) (layer "F.Cu") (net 10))
 (segment (start 158.89 87.3884) (end 159.5374 86.741) (width 0.2) (layer "F.Cu") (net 10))
 (segment (start 158.89 88.365) (end 158.89 87.3884) (width 0.2) (layer "F.Cu") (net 10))
 (via (at 159.8168 83.0834) (size 0.4) (drill 0.2) (layers "F.Cu" "B.Cu") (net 10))
 (via (at 159.5374 86.741) (size 0.4) (drill 0.2) (layers "F.Cu" "B.Cu") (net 10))
 (segment (start 159.8168 86.4616) (end 159.8168 83.0834) (width 0.2) (layer "B.Cu") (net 10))
 (segment (start 159.5374 86.741) (end 159.8168 86.4616) (width 0.2) (layer "B.Cu") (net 10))
 (segment (start 159.39 88.365) (end 159.39 87.6504) (width 0.2) (layer "F.Cu") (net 3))
 (segment (start 158.91 82.9548) (end 158.91 81.965) (width 0.2) (layer "F.Cu") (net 3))
 (segment (start 160.1978 86.8426) (end 160.1978 84.2426) (width 0.2) (layer "F.Cu") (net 3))
 (segment (start 160.1978 84.2426) (end 158.91 82.9548) (width 0.2) (layer "F.Cu") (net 3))
 (segment (start 159.39 87.6504) (end 160.1978 86.8426) (width 0.2) (layer "F.Cu") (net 3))
 (segment (start 157.91 81.965) (end 157.91 84.123) (width 0.2) (layer "F.Cu") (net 4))
 (segment (start 158.39 87.0248) (end 158.39 88.365) (width 0.2) (layer "F.Cu") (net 4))
 (segment (start 157.91 84.123) (end 158.2166 84.4296) (width 0.2) (layer "F.Cu") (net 4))
 (segment (start 158.7246 86.6902) (end 158.39 87.0248) (width 0.2) (layer "F.Cu") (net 4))
 (via (at 158.2166 84.4296) (size 0.4) (drill 0.2) (layers "F.Cu" "B.Cu") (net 4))
 (via (at 158.7246 86.6902) (size 0.4) (drill 0.2) (layers "F.Cu" "B.Cu") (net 4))
 (segment (start 158.2166 84.4296) (end 158.2166 86.1822) (width 0.2) (layer "B.Cu") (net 4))
 (segment (start 158.2166 86.1822) (end 158.7246 86.6902) (width 0.2) (layer "B.Cu") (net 4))
 (segment (start 157.41 84.385) (end 157.41 81.965) (width 0.2) (layer "F.Cu") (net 5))
 (segment (start 157.4292 84.4042) (end 157.41 84.385) (width 0.2) (layer "F.Cu") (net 5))
 (segment (start 156.89 84.9434) (end 157.4292 84.4042) (width 0.2) (layer "F.Cu") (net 5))
 (segment (start 156.89 88.365) (end 156.89 84.9434) (width 0.2) (layer "F.Cu") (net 5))
 (segment (start 155.702 84.2264) (end 155.702 86.8426) (width 0.2) (layer "F.Cu") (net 6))
 (segment (start 156.41 83.5184) (end 155.702 84.2264) (width 0.2) (layer "F.Cu") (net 6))
 (segment (start 155.89 87.0306) (end 155.89 88.365) (width 0.2) (layer "F.Cu") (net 6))
 (segment (start 155.702 86.8426) (end 155.89 87.0306) (width 0.2) (layer "F.Cu") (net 6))
 (segment (start 156.41 81.965) (end 156.41 83.5184) (width 0.2) (layer "F.Cu") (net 6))
 (segment (start 155.11 81.965) (end 155.11 81.44) (width 0.2) (layer "F.Cu") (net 2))
 (segment (start 155.11 81.44) (end 155.46 81.09) (width 0.2) (layer "F.Cu") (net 2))
 (segment (start 161.460507 84.02) (end 169.865 84.02) (width 0.2) (layer "F.Cu") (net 2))
 (segment (start 159.86 81.09) (end 160.21 81.44) (width 0.2) (layer "F.Cu") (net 2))
 (segment (start 160.21 81.965) (end 160.21 82.769493) (width 0.2) (layer "F.Cu") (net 2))
 (segment (start 155.46 81.09) (end 159.86 81.09) (width 0.2) (layer "F.Cu") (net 2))
 (segment (start 160.21 82.769493) (end 161.460507 84.02) (width 0.2) (layer "F.Cu") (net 2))
 (segment (start 160.21 81.44) (end 160.21 81.965) (width 0.2) (layer "F.Cu") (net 2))
 (segment (start 155.09 88.365) (end 155.09 88.79) (width 0.2) (layer "F.Cu") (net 11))
 (segment (start 161.31 86.52) (end 169.865 86.52) (width 0.2) (layer "F.Cu") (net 11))
 (segment (start 155.54 89.24) (end 159.7816 89.24) (width 0.2) (layer "F.Cu") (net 11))
 (segment (start 155.09 88.79) (end 155.54 89.24) (width 0.2) (layer "F.Cu") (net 11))
 (segment (start 159.89 87.94) (end 161.31 86.52) (width 0.2) (layer "F.Cu") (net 11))
 (segment (start 159.89 88.365) (end 159.89 87.94) (width 0.2) (layer "F.Cu") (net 11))
 (segment (start 160.19 88.8316) (end 160.19 88.365) (width 0.2) (layer "F.Cu") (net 11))
 (segment (start 159.7816 89.24) (end 160.19 88.8316) (width 0.2) (layer "F.Cu") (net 11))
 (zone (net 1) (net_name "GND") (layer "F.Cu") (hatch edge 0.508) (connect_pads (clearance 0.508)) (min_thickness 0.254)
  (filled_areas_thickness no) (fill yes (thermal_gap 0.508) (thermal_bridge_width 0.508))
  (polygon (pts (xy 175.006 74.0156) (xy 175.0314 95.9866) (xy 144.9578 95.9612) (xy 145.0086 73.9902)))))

